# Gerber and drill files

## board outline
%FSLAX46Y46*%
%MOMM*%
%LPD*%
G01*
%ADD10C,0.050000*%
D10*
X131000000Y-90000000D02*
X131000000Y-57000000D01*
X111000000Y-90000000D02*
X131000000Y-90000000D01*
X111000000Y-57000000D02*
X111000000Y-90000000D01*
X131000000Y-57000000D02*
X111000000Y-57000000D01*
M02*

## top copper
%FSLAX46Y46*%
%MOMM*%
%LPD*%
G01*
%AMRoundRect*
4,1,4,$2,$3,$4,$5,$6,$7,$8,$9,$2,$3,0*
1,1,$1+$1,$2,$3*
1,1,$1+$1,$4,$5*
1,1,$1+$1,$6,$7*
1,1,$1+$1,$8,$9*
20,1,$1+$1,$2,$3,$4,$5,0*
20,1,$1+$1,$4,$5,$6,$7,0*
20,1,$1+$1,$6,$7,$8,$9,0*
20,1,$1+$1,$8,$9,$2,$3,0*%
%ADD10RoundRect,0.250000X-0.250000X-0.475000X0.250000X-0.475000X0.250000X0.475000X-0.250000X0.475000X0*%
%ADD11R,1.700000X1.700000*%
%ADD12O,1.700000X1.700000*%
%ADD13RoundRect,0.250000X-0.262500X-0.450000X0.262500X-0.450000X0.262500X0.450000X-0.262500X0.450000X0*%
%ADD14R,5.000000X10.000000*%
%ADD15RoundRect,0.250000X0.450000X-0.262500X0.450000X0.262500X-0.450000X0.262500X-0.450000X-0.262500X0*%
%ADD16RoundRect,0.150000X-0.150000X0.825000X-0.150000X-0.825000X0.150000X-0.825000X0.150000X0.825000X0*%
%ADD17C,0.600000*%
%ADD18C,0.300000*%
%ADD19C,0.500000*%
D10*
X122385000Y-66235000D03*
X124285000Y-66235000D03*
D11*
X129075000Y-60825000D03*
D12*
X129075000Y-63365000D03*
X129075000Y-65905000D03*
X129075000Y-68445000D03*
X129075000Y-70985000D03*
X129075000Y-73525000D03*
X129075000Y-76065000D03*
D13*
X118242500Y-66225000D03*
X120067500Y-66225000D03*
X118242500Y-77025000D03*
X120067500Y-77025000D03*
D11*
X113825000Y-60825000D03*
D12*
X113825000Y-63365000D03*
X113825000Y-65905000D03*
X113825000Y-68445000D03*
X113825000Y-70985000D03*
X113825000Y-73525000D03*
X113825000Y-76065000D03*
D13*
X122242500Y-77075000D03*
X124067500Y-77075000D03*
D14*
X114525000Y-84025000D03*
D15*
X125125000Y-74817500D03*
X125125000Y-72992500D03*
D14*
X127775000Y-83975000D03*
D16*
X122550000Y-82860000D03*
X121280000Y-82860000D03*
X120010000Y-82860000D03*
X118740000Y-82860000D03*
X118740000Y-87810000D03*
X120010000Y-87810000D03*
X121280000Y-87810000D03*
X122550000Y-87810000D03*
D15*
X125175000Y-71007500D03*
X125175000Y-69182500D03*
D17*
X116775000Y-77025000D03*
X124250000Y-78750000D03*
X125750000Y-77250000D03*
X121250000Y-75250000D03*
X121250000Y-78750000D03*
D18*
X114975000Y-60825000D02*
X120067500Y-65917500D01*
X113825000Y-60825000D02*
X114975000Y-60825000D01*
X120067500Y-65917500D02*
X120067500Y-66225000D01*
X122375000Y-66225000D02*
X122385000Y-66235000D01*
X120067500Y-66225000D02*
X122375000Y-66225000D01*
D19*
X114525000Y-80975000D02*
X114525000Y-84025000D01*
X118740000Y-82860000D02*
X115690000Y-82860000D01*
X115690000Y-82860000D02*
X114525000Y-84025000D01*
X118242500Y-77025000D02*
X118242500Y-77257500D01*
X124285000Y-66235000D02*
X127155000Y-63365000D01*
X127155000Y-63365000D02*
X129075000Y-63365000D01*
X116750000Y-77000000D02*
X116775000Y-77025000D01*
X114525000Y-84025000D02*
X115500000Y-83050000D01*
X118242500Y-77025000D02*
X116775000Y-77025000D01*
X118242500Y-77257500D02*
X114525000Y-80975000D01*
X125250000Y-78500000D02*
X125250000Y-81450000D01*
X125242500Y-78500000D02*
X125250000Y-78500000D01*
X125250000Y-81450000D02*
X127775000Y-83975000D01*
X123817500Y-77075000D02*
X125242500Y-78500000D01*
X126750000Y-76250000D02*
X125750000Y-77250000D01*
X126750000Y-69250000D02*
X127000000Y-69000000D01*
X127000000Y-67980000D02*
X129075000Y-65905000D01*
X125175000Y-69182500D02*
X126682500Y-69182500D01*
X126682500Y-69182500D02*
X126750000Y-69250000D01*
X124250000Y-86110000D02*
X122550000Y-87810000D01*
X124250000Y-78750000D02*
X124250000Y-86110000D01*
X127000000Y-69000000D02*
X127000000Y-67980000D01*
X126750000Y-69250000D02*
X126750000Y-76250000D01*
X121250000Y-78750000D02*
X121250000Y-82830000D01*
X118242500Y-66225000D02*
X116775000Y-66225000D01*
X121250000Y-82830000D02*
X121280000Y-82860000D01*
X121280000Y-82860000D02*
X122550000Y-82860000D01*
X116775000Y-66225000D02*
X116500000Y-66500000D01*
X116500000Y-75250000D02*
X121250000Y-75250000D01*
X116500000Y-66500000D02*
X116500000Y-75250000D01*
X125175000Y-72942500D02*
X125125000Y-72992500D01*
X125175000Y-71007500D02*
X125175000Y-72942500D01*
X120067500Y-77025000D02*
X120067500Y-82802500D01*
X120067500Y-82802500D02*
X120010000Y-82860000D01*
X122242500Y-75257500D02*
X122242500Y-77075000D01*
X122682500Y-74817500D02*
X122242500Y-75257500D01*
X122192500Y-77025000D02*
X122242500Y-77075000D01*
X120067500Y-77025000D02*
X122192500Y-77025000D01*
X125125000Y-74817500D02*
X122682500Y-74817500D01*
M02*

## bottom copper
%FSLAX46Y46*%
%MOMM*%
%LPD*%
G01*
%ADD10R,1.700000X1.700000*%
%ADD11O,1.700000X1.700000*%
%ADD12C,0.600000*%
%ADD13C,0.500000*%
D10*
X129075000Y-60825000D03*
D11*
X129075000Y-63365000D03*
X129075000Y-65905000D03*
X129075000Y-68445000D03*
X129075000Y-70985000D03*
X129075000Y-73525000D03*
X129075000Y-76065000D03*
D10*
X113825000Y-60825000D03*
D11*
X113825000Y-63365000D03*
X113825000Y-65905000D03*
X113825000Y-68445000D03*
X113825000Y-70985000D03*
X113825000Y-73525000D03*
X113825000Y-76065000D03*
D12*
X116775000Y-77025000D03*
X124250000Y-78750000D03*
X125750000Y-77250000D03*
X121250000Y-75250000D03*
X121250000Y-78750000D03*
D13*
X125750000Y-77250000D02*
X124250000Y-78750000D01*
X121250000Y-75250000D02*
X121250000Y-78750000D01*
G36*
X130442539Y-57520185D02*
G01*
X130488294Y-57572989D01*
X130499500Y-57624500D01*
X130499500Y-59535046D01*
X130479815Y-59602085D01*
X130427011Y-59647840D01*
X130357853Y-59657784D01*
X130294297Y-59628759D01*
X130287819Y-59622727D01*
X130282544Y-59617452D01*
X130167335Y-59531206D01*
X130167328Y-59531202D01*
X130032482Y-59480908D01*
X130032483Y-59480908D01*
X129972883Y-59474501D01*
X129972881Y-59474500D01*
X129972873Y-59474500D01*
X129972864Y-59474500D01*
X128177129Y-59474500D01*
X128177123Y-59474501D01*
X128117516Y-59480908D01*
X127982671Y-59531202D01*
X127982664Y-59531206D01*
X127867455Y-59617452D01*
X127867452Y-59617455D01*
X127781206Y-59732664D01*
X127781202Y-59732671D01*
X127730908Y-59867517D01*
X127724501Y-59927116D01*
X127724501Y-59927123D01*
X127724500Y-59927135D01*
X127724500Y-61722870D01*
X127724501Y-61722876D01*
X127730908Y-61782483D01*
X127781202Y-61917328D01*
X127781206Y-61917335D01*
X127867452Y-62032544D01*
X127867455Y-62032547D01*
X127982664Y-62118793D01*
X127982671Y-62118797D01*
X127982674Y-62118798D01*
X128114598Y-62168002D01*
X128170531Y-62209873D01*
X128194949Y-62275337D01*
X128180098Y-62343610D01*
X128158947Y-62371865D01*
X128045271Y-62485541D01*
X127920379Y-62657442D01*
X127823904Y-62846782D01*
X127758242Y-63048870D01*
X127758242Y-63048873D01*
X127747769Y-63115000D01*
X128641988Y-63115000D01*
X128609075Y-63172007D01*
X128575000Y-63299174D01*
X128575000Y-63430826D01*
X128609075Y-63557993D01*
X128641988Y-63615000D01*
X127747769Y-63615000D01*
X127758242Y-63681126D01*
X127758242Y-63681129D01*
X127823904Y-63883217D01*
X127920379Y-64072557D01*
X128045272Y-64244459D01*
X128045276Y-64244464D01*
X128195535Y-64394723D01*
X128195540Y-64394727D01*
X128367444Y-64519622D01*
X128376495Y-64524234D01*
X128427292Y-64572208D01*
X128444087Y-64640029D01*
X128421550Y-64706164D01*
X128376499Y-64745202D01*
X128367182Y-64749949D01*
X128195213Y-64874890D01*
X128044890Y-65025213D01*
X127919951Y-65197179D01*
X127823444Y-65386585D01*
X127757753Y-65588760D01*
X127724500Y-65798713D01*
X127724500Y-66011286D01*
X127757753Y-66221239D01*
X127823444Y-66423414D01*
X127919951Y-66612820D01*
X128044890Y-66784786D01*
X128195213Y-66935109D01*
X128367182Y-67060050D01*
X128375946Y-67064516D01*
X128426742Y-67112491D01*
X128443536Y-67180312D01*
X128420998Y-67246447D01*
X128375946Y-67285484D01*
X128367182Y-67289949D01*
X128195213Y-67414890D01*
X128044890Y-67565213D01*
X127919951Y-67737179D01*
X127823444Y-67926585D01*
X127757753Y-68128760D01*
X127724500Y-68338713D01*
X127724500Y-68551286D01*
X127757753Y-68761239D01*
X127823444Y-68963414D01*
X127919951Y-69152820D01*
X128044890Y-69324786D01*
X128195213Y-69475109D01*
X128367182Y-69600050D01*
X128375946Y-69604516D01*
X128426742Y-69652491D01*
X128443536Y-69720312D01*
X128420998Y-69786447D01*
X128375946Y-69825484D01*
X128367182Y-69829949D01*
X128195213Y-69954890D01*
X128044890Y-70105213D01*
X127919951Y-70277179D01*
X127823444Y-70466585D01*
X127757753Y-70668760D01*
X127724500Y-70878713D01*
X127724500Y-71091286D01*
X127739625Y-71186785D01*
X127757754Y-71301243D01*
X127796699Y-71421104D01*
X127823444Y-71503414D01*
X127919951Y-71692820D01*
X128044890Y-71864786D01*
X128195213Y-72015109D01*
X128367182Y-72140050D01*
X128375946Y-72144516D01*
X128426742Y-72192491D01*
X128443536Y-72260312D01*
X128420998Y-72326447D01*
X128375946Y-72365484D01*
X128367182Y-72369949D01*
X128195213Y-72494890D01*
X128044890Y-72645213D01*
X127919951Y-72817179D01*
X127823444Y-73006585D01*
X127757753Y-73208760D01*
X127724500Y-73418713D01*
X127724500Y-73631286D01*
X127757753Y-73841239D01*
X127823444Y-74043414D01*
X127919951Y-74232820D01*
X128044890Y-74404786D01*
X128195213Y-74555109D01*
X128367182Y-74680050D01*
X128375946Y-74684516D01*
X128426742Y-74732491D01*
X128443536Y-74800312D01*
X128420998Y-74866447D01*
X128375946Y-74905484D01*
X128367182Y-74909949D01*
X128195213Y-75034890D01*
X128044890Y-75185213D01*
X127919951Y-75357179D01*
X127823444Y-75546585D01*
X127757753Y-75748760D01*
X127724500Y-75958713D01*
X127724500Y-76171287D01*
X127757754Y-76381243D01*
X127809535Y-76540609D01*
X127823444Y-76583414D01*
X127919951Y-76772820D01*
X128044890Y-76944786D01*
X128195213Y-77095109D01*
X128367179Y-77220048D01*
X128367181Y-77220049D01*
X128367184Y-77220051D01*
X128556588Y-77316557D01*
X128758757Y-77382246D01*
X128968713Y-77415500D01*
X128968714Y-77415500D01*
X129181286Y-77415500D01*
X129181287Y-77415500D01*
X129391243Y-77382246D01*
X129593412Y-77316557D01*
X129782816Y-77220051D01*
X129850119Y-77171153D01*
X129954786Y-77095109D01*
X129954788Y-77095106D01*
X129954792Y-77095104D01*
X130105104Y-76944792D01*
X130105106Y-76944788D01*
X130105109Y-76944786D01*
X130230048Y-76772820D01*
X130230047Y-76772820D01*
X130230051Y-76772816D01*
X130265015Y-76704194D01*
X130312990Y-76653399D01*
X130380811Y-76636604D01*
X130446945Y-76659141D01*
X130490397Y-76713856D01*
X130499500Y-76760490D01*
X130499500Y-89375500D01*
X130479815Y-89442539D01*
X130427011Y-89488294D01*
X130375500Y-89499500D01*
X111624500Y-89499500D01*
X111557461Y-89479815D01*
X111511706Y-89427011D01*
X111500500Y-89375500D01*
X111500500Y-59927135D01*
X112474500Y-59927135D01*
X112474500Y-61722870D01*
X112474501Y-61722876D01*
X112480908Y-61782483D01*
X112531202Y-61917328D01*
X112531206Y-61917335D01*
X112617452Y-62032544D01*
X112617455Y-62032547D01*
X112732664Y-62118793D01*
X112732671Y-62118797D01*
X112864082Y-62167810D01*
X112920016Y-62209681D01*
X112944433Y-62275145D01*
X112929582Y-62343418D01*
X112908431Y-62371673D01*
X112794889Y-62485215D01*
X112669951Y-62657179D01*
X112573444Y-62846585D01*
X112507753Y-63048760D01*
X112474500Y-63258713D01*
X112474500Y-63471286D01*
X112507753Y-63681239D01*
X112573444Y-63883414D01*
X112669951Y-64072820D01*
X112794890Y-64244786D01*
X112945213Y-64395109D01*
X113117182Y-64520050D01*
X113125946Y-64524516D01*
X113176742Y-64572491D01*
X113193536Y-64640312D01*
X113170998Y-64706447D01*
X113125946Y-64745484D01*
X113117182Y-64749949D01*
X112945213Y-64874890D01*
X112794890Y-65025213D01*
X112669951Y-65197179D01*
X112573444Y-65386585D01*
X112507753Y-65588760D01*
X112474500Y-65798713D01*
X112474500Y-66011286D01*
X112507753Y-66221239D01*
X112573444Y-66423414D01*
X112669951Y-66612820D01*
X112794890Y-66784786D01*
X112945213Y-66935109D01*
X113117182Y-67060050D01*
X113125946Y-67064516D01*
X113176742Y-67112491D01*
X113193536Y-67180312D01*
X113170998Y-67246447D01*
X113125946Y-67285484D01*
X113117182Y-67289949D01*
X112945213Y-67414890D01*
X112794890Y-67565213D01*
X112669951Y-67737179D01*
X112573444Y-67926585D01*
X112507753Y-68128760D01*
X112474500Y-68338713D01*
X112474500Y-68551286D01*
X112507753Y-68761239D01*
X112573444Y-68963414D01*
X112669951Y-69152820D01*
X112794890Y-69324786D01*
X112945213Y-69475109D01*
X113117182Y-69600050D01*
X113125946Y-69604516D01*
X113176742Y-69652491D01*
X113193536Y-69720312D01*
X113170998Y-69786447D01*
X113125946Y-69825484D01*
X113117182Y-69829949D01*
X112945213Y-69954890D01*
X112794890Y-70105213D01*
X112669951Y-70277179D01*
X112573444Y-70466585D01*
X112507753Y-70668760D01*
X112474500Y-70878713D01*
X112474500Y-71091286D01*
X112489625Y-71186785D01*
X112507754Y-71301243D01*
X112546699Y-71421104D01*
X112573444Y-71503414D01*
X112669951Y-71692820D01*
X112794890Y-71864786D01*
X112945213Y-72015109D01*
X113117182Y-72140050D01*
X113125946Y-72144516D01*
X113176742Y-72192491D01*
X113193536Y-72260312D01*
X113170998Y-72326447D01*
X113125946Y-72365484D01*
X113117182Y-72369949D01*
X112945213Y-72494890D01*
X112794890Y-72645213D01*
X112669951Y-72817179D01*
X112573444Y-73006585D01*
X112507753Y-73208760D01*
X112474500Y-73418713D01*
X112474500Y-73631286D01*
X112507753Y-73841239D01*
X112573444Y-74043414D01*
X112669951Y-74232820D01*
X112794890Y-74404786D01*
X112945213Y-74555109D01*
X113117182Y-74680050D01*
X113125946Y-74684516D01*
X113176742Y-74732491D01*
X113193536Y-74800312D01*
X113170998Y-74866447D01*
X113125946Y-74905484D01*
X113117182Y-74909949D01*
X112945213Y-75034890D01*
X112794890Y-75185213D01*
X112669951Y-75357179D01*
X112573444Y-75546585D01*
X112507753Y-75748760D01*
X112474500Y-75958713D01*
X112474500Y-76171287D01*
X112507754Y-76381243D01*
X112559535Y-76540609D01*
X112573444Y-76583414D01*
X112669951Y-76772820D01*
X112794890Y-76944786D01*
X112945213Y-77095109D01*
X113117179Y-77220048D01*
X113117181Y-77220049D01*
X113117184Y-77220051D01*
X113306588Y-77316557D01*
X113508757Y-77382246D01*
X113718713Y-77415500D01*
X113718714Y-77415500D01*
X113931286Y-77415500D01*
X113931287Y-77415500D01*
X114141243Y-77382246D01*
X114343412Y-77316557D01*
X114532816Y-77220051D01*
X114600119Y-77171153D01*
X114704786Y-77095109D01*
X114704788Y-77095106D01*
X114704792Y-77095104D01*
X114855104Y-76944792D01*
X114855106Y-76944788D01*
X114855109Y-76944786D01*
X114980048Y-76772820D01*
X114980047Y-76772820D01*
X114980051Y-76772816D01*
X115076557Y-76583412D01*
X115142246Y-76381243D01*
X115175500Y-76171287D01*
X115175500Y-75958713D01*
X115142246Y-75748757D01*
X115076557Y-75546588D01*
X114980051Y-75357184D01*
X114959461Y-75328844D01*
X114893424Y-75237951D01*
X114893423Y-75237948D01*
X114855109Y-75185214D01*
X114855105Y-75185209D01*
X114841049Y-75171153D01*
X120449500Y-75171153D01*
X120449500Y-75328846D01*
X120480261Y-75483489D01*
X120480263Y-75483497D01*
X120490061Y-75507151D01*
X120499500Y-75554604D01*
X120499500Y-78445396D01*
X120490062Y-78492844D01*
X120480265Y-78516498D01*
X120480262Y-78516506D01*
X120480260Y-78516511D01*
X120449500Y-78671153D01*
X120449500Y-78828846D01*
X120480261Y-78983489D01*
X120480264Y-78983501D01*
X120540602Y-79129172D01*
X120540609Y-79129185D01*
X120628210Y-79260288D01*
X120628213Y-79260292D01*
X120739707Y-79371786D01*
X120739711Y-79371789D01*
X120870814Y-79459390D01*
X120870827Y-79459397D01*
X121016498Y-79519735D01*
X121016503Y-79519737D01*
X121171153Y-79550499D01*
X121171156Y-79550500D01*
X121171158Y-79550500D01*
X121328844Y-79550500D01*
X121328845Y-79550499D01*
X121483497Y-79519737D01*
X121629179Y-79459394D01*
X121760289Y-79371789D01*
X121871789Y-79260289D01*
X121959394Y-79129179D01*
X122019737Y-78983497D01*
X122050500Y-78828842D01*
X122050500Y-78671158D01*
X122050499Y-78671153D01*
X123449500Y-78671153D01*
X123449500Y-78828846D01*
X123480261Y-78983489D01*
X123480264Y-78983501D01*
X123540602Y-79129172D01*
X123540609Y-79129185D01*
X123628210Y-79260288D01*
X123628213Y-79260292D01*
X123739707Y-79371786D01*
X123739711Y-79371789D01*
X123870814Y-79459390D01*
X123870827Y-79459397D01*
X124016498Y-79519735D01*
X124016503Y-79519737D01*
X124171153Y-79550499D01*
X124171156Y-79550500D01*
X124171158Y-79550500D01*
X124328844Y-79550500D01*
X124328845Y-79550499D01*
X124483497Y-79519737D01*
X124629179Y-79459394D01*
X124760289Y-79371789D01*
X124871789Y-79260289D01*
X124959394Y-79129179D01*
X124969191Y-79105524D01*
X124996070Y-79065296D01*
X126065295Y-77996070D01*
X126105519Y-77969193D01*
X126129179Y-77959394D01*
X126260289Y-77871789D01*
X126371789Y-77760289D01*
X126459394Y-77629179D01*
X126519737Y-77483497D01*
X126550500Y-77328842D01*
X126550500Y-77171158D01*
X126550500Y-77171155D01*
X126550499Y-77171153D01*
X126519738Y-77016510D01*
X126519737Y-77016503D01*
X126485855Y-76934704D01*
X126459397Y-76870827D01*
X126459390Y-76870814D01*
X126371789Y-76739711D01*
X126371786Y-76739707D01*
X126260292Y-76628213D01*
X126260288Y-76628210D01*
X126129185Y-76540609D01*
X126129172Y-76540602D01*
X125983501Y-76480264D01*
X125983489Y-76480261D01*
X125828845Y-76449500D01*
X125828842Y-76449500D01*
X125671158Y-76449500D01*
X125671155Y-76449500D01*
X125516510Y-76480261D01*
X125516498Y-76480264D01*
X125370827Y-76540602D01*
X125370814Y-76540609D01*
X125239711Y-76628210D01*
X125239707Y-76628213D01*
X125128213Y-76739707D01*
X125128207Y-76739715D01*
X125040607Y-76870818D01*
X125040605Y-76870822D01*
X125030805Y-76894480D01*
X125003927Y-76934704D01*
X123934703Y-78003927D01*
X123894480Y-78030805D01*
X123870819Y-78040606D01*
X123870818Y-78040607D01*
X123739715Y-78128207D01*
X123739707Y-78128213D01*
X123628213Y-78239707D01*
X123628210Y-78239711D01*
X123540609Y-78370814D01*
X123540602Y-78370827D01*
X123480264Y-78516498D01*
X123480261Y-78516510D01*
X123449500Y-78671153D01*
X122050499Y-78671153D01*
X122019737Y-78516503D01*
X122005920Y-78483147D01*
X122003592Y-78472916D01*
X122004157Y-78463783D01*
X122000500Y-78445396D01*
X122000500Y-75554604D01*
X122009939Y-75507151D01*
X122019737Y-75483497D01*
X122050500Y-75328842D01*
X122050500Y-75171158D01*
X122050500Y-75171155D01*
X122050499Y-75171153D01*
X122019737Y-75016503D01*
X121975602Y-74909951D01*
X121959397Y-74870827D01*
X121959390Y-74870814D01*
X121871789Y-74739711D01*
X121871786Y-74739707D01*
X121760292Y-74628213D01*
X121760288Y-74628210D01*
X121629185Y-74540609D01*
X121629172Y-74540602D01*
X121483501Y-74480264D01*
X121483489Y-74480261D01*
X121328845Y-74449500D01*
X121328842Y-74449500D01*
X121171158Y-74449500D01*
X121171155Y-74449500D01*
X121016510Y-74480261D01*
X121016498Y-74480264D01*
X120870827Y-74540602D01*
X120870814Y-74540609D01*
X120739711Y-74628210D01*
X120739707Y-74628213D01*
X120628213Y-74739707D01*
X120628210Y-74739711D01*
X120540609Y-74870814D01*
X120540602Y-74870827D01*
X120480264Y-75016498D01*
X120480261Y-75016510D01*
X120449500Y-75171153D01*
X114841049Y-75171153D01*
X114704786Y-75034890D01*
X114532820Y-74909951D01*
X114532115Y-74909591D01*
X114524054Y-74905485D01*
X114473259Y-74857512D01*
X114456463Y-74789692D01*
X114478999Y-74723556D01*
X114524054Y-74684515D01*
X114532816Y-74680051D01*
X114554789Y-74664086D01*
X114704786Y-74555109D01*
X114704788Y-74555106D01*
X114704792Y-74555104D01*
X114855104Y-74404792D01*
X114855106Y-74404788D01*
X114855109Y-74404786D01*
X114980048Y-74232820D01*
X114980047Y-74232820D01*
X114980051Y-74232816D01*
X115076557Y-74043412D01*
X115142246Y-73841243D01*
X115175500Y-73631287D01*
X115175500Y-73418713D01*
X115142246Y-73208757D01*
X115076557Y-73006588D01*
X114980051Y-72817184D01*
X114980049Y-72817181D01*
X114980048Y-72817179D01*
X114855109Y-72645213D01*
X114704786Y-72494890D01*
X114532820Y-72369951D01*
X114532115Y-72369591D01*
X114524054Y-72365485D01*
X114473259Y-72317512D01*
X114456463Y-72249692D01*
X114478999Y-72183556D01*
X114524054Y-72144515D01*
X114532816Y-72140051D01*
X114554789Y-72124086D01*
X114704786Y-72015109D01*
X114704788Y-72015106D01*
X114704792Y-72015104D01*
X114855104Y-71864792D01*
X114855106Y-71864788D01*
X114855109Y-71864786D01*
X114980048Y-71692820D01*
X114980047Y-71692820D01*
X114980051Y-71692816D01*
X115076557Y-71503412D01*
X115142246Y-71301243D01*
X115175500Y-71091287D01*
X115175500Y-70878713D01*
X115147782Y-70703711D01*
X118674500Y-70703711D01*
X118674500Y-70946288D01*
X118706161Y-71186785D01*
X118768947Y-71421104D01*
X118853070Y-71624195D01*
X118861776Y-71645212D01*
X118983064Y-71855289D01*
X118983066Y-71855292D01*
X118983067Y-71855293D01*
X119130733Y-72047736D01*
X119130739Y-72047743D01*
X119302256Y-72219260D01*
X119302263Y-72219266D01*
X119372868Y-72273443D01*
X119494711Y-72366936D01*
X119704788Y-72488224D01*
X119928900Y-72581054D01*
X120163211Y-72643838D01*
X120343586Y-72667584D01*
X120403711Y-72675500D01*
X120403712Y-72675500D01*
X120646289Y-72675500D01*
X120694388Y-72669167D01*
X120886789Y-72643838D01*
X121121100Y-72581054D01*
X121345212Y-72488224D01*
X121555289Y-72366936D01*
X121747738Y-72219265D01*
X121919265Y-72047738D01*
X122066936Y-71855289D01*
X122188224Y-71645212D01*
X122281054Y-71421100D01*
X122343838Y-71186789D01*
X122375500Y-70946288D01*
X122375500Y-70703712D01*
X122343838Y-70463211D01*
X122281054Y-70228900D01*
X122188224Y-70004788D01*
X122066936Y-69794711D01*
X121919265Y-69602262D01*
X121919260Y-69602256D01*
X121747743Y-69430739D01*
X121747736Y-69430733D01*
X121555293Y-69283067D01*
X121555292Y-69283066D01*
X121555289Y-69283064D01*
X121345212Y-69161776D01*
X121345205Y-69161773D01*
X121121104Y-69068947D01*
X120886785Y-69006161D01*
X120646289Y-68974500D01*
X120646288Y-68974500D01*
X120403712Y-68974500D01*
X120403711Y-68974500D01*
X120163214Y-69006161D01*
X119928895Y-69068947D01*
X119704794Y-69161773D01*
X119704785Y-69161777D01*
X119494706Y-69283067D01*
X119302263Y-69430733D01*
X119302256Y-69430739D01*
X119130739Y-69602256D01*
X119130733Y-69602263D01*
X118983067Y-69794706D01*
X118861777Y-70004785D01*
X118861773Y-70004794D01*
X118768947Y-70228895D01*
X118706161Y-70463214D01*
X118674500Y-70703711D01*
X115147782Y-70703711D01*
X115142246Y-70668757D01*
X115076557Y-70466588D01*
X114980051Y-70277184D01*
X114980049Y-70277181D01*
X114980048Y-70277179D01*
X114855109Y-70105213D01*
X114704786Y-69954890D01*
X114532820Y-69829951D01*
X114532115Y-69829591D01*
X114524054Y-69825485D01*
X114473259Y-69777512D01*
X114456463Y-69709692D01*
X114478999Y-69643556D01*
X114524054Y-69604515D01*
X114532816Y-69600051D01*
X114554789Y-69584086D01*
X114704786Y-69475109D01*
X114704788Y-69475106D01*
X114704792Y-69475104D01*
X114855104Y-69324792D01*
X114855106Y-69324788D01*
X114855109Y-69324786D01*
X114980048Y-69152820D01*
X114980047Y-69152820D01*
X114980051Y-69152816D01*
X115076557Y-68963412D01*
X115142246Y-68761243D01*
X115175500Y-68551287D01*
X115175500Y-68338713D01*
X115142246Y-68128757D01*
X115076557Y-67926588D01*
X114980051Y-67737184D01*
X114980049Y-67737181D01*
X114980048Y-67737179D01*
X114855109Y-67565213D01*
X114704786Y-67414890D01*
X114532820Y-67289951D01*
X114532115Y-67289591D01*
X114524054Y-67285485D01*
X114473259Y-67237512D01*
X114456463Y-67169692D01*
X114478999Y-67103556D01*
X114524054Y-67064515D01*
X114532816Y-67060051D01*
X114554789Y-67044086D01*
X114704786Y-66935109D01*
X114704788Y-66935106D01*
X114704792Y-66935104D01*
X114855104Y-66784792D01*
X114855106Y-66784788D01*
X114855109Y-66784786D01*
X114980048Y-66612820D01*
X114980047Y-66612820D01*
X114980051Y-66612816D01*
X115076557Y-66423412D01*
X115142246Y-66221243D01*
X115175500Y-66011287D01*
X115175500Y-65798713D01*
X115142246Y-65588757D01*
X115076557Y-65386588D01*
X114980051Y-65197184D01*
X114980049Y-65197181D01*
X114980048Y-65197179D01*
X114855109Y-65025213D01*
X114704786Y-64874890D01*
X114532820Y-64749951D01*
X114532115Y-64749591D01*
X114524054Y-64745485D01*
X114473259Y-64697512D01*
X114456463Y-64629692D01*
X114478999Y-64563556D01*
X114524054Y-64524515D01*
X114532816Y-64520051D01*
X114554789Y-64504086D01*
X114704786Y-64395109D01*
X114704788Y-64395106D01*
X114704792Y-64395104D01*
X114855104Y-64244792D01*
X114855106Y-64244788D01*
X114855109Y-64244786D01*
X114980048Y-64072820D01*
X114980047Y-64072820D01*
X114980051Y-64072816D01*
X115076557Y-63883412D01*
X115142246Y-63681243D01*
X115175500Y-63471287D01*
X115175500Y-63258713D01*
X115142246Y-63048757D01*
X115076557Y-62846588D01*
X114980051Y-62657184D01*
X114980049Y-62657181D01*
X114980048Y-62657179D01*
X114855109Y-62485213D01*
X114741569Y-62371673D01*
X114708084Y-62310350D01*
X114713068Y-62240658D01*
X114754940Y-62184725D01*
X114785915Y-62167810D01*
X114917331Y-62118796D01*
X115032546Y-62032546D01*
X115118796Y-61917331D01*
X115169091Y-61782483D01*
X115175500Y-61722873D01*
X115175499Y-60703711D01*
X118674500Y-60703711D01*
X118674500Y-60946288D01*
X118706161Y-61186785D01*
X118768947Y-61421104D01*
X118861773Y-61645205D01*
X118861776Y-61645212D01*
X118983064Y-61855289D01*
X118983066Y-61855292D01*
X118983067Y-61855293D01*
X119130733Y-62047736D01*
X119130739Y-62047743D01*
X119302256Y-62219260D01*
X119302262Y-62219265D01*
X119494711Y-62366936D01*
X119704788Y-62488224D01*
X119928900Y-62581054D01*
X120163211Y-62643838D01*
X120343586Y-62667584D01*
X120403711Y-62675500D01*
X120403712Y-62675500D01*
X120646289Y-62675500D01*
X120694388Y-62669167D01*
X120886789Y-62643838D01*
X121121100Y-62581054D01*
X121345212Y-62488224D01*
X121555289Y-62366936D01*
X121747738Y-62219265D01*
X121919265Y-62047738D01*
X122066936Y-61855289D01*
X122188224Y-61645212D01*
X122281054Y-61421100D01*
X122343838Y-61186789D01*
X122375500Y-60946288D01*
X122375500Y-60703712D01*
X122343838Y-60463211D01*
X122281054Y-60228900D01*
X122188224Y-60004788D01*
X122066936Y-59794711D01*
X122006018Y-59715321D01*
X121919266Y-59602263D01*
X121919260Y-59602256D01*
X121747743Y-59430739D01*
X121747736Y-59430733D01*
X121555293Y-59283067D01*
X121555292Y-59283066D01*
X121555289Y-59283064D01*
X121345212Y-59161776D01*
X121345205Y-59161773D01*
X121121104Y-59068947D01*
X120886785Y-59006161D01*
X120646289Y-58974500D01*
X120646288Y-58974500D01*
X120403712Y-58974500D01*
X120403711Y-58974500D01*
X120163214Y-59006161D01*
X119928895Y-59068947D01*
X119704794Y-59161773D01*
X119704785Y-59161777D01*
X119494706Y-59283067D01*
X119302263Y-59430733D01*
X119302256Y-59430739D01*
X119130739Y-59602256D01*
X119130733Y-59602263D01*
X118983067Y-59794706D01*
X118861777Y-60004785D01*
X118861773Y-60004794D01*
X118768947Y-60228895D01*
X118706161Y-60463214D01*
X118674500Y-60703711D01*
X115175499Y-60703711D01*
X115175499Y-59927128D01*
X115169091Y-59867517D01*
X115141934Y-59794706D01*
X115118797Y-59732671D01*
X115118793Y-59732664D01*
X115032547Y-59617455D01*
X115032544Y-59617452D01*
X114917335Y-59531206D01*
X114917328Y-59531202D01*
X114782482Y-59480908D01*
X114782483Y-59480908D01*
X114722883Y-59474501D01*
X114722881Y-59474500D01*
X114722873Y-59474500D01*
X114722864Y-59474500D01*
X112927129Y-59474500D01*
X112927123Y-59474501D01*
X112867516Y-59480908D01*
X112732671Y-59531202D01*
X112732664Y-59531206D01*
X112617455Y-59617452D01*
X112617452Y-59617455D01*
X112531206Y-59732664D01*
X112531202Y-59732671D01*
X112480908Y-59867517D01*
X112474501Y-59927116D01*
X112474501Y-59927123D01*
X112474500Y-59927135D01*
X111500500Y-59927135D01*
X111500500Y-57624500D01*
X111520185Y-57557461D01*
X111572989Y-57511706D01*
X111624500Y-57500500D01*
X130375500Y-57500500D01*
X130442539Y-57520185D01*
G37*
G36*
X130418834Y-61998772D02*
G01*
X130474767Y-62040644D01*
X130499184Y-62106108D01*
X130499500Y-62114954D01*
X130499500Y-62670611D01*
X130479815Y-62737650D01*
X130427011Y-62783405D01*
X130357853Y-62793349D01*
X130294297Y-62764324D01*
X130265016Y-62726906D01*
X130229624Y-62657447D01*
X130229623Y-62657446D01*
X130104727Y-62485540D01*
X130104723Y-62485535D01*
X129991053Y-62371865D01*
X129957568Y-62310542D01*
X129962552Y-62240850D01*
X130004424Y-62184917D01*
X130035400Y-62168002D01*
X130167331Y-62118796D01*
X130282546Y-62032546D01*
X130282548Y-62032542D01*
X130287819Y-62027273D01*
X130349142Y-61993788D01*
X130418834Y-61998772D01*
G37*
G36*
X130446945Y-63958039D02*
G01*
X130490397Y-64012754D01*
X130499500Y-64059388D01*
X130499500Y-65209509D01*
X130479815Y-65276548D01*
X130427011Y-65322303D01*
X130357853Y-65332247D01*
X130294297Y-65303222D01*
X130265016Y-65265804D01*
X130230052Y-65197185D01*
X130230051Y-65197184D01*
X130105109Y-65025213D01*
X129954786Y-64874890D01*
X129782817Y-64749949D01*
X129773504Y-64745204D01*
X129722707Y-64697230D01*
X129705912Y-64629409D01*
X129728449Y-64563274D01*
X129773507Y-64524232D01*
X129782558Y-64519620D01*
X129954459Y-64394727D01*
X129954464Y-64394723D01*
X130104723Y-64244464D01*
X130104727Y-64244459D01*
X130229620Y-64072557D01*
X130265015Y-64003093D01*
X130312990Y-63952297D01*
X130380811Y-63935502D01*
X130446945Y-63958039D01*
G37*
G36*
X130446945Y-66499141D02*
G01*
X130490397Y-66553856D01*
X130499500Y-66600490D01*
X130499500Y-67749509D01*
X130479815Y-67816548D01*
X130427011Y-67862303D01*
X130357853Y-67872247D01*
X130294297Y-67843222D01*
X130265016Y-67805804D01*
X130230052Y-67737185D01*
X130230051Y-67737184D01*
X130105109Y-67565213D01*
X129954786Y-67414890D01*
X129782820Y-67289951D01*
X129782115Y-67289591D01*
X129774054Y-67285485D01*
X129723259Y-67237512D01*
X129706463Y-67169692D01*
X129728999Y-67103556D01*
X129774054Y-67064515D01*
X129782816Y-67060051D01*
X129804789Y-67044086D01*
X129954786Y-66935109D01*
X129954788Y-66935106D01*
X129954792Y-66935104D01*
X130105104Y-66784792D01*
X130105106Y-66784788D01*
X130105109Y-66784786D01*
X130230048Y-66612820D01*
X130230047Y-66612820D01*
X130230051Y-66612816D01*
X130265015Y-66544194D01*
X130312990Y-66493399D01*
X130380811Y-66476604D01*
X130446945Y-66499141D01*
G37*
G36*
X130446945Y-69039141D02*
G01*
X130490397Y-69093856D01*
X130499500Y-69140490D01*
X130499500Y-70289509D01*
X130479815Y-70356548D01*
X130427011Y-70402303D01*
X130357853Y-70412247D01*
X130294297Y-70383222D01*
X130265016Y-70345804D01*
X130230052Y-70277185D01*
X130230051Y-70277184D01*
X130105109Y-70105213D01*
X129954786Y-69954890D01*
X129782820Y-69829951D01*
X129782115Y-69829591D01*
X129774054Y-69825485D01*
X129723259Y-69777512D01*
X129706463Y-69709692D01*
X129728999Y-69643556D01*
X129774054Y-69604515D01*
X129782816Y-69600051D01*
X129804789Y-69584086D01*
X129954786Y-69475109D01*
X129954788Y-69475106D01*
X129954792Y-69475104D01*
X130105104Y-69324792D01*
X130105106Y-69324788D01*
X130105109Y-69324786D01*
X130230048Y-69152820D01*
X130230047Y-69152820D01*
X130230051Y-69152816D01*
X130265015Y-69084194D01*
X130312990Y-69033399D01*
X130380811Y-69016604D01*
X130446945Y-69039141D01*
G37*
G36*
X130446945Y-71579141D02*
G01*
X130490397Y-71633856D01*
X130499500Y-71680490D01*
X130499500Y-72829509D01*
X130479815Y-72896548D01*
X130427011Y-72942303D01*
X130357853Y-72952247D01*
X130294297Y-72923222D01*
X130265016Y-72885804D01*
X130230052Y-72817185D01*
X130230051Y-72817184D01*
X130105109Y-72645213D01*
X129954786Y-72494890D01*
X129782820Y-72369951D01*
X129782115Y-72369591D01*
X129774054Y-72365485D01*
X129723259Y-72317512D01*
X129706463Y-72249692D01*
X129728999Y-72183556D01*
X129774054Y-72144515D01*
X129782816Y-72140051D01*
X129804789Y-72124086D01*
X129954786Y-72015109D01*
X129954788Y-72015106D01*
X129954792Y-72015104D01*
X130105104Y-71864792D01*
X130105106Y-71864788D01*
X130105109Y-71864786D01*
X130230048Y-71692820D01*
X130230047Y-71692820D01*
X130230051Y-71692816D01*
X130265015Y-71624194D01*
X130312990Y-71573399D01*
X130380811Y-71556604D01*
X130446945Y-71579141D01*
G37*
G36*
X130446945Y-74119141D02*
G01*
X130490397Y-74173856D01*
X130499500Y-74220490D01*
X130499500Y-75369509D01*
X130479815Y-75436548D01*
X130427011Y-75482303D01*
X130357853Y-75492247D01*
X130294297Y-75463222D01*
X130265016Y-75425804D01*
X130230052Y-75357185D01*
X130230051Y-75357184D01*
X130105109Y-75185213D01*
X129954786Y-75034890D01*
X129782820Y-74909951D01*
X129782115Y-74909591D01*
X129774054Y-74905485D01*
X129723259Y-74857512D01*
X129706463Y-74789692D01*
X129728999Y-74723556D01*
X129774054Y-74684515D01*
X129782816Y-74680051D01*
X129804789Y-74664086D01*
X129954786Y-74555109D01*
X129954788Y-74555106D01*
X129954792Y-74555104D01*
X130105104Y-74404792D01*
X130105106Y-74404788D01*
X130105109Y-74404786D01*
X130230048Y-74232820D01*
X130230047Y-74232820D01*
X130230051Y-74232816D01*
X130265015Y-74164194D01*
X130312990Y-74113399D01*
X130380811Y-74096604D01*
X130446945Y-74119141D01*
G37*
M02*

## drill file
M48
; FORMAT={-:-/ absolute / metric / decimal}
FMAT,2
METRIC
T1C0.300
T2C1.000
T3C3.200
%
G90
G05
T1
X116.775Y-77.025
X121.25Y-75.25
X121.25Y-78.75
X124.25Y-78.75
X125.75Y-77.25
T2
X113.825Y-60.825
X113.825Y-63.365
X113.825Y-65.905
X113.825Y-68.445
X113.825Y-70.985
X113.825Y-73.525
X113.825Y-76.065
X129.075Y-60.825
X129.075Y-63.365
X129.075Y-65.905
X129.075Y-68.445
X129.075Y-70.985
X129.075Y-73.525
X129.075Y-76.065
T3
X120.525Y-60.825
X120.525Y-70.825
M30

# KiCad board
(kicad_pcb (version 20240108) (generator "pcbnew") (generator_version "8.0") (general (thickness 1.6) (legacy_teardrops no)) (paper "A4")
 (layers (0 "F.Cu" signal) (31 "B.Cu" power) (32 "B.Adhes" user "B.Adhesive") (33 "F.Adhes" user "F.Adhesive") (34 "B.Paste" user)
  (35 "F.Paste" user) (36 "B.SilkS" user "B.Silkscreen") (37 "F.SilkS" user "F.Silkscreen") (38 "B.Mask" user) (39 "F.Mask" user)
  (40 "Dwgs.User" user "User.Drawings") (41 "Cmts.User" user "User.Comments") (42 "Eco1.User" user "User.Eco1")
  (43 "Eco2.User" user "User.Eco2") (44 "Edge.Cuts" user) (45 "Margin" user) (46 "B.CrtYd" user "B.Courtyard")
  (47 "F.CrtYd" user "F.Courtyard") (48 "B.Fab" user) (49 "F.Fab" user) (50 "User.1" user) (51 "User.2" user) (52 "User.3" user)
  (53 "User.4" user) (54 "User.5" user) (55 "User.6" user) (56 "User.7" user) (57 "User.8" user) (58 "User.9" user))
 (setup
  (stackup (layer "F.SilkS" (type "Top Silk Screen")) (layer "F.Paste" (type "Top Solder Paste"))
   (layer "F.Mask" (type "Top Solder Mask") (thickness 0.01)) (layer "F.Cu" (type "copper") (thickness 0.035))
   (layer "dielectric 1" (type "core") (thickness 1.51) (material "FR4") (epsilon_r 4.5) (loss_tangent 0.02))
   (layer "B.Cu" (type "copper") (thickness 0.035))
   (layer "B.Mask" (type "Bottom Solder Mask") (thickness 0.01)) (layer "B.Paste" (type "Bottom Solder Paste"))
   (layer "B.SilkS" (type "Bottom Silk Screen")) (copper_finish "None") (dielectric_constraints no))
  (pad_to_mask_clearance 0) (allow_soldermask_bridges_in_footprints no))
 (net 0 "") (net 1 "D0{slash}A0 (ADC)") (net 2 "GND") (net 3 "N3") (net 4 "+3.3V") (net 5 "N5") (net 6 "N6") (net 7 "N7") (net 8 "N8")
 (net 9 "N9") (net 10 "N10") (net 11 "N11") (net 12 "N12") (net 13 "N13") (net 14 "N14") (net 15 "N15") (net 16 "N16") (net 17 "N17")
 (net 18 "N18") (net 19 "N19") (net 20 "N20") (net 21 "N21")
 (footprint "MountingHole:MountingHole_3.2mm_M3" (layer "F.Cu") (at 120.525 60.825)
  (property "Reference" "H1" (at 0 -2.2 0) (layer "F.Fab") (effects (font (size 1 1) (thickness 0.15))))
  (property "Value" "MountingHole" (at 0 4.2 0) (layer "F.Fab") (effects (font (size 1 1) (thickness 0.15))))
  (pad "" np_thru_hole circle (at 0 0) (size 3.2 3.2) (drill 3.2) (layers "*.Cu" "*.Mask")))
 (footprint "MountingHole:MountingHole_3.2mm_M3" (layer "F.Cu") (at 120.525 70.825)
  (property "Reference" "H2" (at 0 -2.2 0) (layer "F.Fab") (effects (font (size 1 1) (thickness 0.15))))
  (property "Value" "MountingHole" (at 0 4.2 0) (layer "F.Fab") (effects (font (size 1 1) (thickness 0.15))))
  (pad "" np_thru_hole circle (at 0 0) (size 3.2 3.2) (drill 3.2) (layers "*.Cu" "*.Mask")))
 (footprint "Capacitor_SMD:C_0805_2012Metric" (layer "F.Cu") (at 123.335 66.235)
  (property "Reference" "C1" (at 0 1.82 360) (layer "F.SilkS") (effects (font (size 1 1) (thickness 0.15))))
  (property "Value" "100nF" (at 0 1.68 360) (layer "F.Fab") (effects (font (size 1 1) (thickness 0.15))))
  (pad "1" smd roundrect (at -0.95 0) (size 1 1.45) (layers "F.Cu" "F.Paste" "F.Mask") (roundrect_rratio 0.25) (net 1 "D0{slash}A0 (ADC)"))
  (pad "2" smd roundrect (at 0.95 0) (size 1 1.45) (layers "F.Cu" "F.Paste" "F.Mask") (roundrect_rratio 0.25) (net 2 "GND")))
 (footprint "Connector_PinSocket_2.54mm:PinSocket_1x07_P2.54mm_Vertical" (layer "F.Cu") (at 129.075 60.825)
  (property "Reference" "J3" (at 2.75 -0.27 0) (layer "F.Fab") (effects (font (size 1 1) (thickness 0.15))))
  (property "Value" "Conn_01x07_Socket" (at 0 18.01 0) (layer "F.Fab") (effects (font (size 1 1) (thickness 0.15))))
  (pad "1" thru_hole rect (at 0 0) (size 1.7 1.7) (drill 1) (layers "*.Cu" "*.Mask") (remove_unused_layers no) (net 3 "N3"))
  (pad "2" thru_hole oval (at 0 2.54) (size 1.7 1.7) (drill 1) (layers "*.Cu" "*.Mask") (remove_unused_layers no) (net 2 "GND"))
  (pad "3" thru_hole oval (at 0 5.08) (size 1.7 1.7) (drill 1) (layers "*.Cu" "*.Mask") (remove_unused_layers no) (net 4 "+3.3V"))
  (pad "4" thru_hole oval (at 0 7.62) (size 1.7 1.7) (drill 1) (layers "*.Cu" "*.Mask") (remove_unused_layers no) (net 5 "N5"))
  (pad "5" thru_hole oval (at 0 10.16) (size 1.7 1.7) (drill 1) (layers "*.Cu" "*.Mask") (remove_unused_layers no) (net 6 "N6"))
  (pad "6" thru_hole oval (at 0 12.7) (size 1.7 1.7) (drill 1) (layers "*.Cu" "*.Mask") (remove_unused_layers no) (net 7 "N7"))
  (pad "7" thru_hole oval (at 0 15.24) (size 1.7 1.7) (drill 1) (layers "*.Cu" "*.Mask") (remove_unused_layers no) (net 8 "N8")))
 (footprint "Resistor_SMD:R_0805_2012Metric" (layer "F.Cu") (at 119.155 66.225)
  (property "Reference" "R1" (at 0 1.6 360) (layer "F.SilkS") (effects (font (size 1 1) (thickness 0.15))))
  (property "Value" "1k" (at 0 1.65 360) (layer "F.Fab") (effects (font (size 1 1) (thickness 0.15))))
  (pad "1" smd roundrect (at -0.9125 0) (size 1.025 1.4) (layers "F.Cu" "F.Paste" "F.Mask") (roundrect_rratio 0.243902) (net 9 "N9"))
  (pad "2" smd roundrect (at 0.9125 0) (size 1.025 1.4) (layers "F.Cu" "F.Paste" "F.Mask") (roundrect_rratio 0.243902)
   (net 1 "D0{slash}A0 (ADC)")))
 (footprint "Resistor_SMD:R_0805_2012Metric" (layer "F.Cu") (at 119.155 77.025)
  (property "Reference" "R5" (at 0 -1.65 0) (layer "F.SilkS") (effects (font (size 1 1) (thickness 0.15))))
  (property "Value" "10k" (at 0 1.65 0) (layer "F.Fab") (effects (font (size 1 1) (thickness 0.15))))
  (pad "1" smd roundrect (at -0.9125 0) (size 1.025 1.4) (layers "F.Cu" "F.Paste" "F.Mask") (roundrect_rratio 0.243902) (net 2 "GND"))
  (pad "2" smd roundrect (at 0.9125 0) (size 1.025 1.4) (layers "F.Cu" "F.Paste" "F.Mask") (roundrect_rratio 0.243902) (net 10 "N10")))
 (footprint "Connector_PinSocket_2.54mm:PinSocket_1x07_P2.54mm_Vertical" (layer "F.Cu") (at 113.825 60.825)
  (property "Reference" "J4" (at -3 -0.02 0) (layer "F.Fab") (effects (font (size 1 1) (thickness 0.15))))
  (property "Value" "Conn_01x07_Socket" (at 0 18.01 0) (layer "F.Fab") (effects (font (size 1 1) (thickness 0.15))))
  (pad "1" thru_hole rect (at 0 0) (size 1.7 1.7) (drill 1) (layers "*.Cu" "*.Mask") (remove_unused_layers no) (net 1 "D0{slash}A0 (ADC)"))
  (pad "2" thru_hole oval (at 0 2.54) (size 1.7 1.7) (drill 1) (layers "*.Cu" "*.Mask") (remove_unused_layers no) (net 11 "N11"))
  (pad "3" thru_hole oval (at 0 5.08) (size 1.7 1.7) (drill 1) (layers "*.Cu" "*.Mask") (remove_unused_layers no) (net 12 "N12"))
  (pad "4" thru_hole oval (at 0 7.62) (size 1.7 1.7) (drill 1) (layers "*.Cu" "*.Mask") (remove_unused_layers no) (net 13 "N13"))
  (pad "5" thru_hole oval (at 0 10.16) (size 1.7 1.7) (drill 1) (layers "*.Cu" "*.Mask") (remove_unused_layers no) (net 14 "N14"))
  (pad "6" thru_hole oval (at 0 12.7) (size 1.7 1.7) (drill 1) (layers "*.Cu" "*.Mask") (remove_unused_layers no) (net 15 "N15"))
  (pad "7" thru_hole oval (at 0 15.24) (size 1.7 1.7) (drill 1) (layers "*.Cu" "*.Mask") (remove_unused_layers no) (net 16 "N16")))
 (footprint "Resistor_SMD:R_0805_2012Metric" (layer "F.Cu") (at 123.155 77.075)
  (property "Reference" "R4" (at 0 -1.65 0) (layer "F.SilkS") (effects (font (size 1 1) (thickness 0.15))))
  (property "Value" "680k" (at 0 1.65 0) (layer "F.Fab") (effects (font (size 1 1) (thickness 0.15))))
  (pad "1" smd roundrect (at -0.9125 0) (size 1.025 1.4) (layers "F.Cu" "F.Paste" "F.Mask") (roundrect_rratio 0.243902) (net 10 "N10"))
  (pad "2" smd roundrect (at 0.9125 0) (size 1.025 1.4) (layers "F.Cu" "F.Paste" "F.Mask") (roundrect_rratio 0.243902) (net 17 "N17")))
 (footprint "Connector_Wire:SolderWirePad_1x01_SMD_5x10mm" (layer "F.Cu") (at 114.525 84.025)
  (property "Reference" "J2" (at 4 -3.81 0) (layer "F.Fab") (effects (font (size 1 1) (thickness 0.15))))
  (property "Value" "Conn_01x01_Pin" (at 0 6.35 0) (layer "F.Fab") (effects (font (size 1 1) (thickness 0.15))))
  (pad "1" smd rect (at 0 0) (size 5 10) (layers "F.Cu" "F.Paste" "F.Mask") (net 2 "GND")))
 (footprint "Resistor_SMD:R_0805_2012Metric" (layer "F.Cu") (at 125.125 73.905 90)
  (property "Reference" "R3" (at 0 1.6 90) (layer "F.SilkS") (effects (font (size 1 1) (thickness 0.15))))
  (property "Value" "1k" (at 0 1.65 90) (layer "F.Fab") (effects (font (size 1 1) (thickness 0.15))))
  (pad "1" smd roundrect (at -0.9125 0 90) (size 1.025 1.4) (layers "F.Cu" "F.Paste" "F.Mask") (roundrect_rratio 0.243902) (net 10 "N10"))
  (pad "2" smd roundrect (at 0.9125 0 90) (size 1.025 1.4) (layers "F.Cu" "F.Paste" "F.Mask") (roundrect_rratio 0.243902) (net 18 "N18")))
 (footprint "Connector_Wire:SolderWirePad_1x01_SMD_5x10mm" (layer "F.Cu") (at 127.775 83.975 180)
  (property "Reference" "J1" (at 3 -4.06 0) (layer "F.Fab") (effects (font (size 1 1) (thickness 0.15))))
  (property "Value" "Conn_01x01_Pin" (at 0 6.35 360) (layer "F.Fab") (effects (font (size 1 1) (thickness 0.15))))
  (pad "1" smd rect (at 0 0 180) (size 5 10) (layers "F.Cu" "F.Paste" "F.Mask") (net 17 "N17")))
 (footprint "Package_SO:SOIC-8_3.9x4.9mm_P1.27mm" (layer "F.Cu") (at 120.645 85.335 -90)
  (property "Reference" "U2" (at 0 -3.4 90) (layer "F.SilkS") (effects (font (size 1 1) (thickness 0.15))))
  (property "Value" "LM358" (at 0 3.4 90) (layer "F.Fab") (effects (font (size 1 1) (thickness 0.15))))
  (pad "1" smd roundrect (at -2.475 -1.905 270) (size 1.95 0.6) (layers "F.Cu" "F.Paste" "F.Mask") (roundrect_rratio 0.25) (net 9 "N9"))
  (pad "2" smd roundrect (at -2.475 -0.635 270) (size 1.95 0.6) (layers "F.Cu" "F.Paste" "F.Mask") (roundrect_rratio 0.25) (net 9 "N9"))
  (pad "3" smd roundrect (at -2.475 0.635 270) (size 1.95 0.6) (layers "F.Cu" "F.Paste" "F.Mask") (roundrect_rratio 0.25) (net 10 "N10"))
  (pad "4" smd roundrect (at -2.475 1.905 270) (size 1.95 0.6) (layers "F.Cu" "F.Paste" "F.Mask") (roundrect_rratio 0.25) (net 2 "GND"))
  (pad "5" smd roundrect (at 2.475 1.905 270) (size 1.95 0.6) (layers "F.Cu" "F.Paste" "F.Mask") (roundrect_rratio 0.25) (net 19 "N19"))
  (pad "6" smd roundrect (at 2.475 0.635 270) (size 1.95 0.6) (layers "F.Cu" "F.Paste" "F.Mask") (roundrect_rratio 0.25) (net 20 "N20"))
  (pad "7" smd roundrect (at 2.475 -0.635 270) (size 1.95 0.6) (layers "F.Cu" "F.Paste" "F.Mask") (roundrect_rratio 0.25) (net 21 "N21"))
  (pad "8" smd roundrect (at 2.475 -1.905 270) (size 1.95 0.6) (layers "F.Cu" "F.Paste" "F.Mask") (roundrect_rratio 0.25) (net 4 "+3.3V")))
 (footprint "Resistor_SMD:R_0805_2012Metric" (layer "F.Cu") (at 125.175 70.095 90)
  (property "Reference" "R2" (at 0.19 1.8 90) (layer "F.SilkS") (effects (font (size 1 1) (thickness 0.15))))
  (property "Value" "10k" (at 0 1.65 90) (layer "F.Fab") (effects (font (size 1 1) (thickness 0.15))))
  (pad "1" smd roundrect (at -0.9125 0 90) (size 1.025 1.4) (layers "F.Cu" "F.Paste" "F.Mask") (roundrect_rratio 0.243902) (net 18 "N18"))
  (pad "2" smd roundrect (at 0.9125 0 90) (size 1.025 1.4) (layers "F.Cu" "F.Paste" "F.Mask") (roundrect_rratio 0.243902) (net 4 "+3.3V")))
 (gr_line (start 131 90) (end 131 57) (stroke (width 0.05) (type default)) (layer "Edge.Cuts"))
 (gr_line (start 111 90) (end 131 90) (stroke (width 0.05) (type default)) (layer "Edge.Cuts"))
 (gr_line (start 111 57) (end 111 90) (stroke (width 0.05) (type default)) (layer "Edge.Cuts"))
 (gr_line (start 131 57) (end 111 57) (stroke (width 0.05) (type default)) (layer "Edge.Cuts"))
 (segment (start 114.975 60.825) (end 120.0675 65.9175) (width 0.3) (layer "F.Cu") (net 1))
 (segment (start 113.825 60.825) (end 114.975 60.825) (width 0.3) (layer "F.Cu") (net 1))
 (segment (start 120.0675 65.9175) (end 120.0675 66.225) (width 0.3) (layer "F.Cu") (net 1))
 (segment (start 122.375 66.225) (end 122.385 66.235) (width 0.3) (layer "F.Cu") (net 1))
 (segment (start 120.0675 66.225) (end 122.375 66.225) (width 0.3) (layer "F.Cu") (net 1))
 (segment (start 114.525 80.975) (end 114.525 84.025) (width 0.5) (layer "F.Cu") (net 2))
 (segment (start 118.74 82.86) (end 115.69 82.86) (width 0.5) (layer "F.Cu") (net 2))
 (segment (start 115.69 82.86) (end 114.525 84.025) (width 0.5) (layer "F.Cu") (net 2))
 (segment (start 118.2425 77.025) (end 118.2425 77.2575) (width 0.5) (layer "F.Cu") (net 2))
 (segment (start 124.285 66.235) (end 127.155 63.365) (width 0.5) (layer "F.Cu") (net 2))
 (segment (start 127.155 63.365) (end 129.075 63.365) (width 0.5) (layer "F.Cu") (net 2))
 (segment (start 116.75 77) (end 116.775 77.025) (width 0.5) (layer "F.Cu") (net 2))
 (segment (start 114.525 84.025) (end 115.5 83.05) (width 0.5) (layer "F.Cu") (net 2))
 (segment (start 118.2425 77.025) (end 116.775 77.025) (width 0.5) (layer "F.Cu") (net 2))
 (segment (start 118.2425 77.2575) (end 114.525 80.975) (width 0.5) (layer "F.Cu") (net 2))
 (via (at 116.775 77.025) (size 0.6) (drill 0.3) (layers "F.Cu" "B.Cu") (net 2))
 (segment (start 125.25 78.5) (end 125.25 81.45) (width 0.5) (layer "F.Cu") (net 17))
 (segment (start 125.2425 78.5) (end 125.25 78.5) (width 0.5) (layer "F.Cu") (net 17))
 (segment (start 125.25 81.45) (end 127.775 83.975) (width 0.5) (layer "F.Cu") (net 17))
 (segment (start 123.8175 77.075) (end 125.2425 78.5) (width 0.5) (layer "F.Cu") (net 17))
 (segment (start 126.75 76.25) (end 125.75 77.25) (width 0.5) (layer "F.Cu") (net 4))
 (segment (start 126.75 69.25) (end 127 69) (width 0.5) (layer "F.Cu") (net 4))
 (segment (start 127 67.98) (end 129.075 65.905) (width 0.5) (layer "F.Cu") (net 4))
 (segment (start 125.175 69.1825) (end 126.6825 69.1825) (width 0.5) (layer "F.Cu") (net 4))
 (segment (start 126.6825 69.1825) (end 126.75 69.25) (width 0.5) (layer "F.Cu") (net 4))
 (segment (start 124.25 86.11) (end 122.55 87.81) (width 0.5) (layer "F.Cu") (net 4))
 (segment (start 124.25 78.75) (end 124.25 86.11) (width 0.5) (layer "F.Cu") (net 4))
 (segment (start 127 69) (end 127 67.98) (width 0.5) (layer "F.Cu") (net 4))
 (segment (start 126.75 69.25) (end 126.75 76.25) (width 0.5) (layer "F.Cu") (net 4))
 (via (at 124.25 78.75) (size 0.6) (drill 0.3) (layers "F.Cu" "B.Cu") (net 4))
 (via (at 125.75 77.25) (size 0.6) (drill 0.3) (layers "F.Cu" "B.Cu") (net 4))
 (segment (start 125.75 77.25) (end 124.25 78.75) (width 0.5) (layer "B.Cu") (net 4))
 (segment (start 121.25 78.75) (end 121.25 82.83) (width 0.5) (layer "F.Cu") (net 9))
 (segment (start 118.2425 66.225) (end 116.775 66.225) (width 0.5) (layer "F.Cu") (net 9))
 (segment (start 121.25 82.83) (end 121.28 82.86) (width 0.5) (layer "F.Cu") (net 9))
 (segment (start 121.28 82.86) (end 122.55 82.86) (width 0.5) (layer "F.Cu") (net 9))
 (segment (start 116.775 66.225) (end 116.5 66.5) (width 0.5) (layer "F.Cu") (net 9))
 (segment (start 116.5 75.25) (end 121.25 75.25) (width 0.5) (layer "F.Cu") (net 9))
 (segment (start 116.5 66.5) (end 116.5 75.25) (width 0.5) (layer "F.Cu") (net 9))
 (via (at 121.25 75.25) (size 0.6) (drill 0.3) (layers "F.Cu" "B.Cu") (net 9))
 (via (at 121.25 78.75) (size 0.6) (drill 0.3) (layers "F.Cu" "B.Cu") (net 9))
 (segment (start 121.25 75.25) (end 121.25 78.75) (width 0.5) (layer "B.Cu") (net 9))
 (segment (start 125.175 72.9425) (end 125.125 72.9925) (width 0.5) (layer "F.Cu") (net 18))
 (segment (start 125.175 71.0075) (end 125.175 72.9425) (width 0.5) (layer "F.Cu") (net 18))
 (segment (start 120.0675 77.025) (end 120.0675 82.8025) (width 0.5) (layer "F.Cu") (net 10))
 (segment (start 120.0675 82.8025) (end 120.01 82.86) (width 0.5) (layer "F.Cu") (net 10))
 (segment (start 122.2425 75.2575) (end 122.2425 77.075) (width 0.5) (layer "F.Cu") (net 10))
 (segment (start 122.6825 74.8175) (end 122.2425 75.2575) (width 0.5) (layer "F.Cu") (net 10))
 (segment (start 122.1925 77.025) (end 122.2425 77.075) (width 0.5) (layer "F.Cu") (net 10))
 (segment (start 120.0675 77.025) (end 122.1925 77.025) (width 0.5) (layer "F.Cu") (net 10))
 (segment (start 125.125 74.8175) (end 122.6825 74.8175) (width 0.5) (layer "F.Cu") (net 10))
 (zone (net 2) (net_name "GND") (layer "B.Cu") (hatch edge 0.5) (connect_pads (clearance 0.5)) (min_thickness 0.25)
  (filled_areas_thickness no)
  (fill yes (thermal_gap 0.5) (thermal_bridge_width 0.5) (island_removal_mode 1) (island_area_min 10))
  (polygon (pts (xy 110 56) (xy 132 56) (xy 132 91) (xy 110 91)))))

